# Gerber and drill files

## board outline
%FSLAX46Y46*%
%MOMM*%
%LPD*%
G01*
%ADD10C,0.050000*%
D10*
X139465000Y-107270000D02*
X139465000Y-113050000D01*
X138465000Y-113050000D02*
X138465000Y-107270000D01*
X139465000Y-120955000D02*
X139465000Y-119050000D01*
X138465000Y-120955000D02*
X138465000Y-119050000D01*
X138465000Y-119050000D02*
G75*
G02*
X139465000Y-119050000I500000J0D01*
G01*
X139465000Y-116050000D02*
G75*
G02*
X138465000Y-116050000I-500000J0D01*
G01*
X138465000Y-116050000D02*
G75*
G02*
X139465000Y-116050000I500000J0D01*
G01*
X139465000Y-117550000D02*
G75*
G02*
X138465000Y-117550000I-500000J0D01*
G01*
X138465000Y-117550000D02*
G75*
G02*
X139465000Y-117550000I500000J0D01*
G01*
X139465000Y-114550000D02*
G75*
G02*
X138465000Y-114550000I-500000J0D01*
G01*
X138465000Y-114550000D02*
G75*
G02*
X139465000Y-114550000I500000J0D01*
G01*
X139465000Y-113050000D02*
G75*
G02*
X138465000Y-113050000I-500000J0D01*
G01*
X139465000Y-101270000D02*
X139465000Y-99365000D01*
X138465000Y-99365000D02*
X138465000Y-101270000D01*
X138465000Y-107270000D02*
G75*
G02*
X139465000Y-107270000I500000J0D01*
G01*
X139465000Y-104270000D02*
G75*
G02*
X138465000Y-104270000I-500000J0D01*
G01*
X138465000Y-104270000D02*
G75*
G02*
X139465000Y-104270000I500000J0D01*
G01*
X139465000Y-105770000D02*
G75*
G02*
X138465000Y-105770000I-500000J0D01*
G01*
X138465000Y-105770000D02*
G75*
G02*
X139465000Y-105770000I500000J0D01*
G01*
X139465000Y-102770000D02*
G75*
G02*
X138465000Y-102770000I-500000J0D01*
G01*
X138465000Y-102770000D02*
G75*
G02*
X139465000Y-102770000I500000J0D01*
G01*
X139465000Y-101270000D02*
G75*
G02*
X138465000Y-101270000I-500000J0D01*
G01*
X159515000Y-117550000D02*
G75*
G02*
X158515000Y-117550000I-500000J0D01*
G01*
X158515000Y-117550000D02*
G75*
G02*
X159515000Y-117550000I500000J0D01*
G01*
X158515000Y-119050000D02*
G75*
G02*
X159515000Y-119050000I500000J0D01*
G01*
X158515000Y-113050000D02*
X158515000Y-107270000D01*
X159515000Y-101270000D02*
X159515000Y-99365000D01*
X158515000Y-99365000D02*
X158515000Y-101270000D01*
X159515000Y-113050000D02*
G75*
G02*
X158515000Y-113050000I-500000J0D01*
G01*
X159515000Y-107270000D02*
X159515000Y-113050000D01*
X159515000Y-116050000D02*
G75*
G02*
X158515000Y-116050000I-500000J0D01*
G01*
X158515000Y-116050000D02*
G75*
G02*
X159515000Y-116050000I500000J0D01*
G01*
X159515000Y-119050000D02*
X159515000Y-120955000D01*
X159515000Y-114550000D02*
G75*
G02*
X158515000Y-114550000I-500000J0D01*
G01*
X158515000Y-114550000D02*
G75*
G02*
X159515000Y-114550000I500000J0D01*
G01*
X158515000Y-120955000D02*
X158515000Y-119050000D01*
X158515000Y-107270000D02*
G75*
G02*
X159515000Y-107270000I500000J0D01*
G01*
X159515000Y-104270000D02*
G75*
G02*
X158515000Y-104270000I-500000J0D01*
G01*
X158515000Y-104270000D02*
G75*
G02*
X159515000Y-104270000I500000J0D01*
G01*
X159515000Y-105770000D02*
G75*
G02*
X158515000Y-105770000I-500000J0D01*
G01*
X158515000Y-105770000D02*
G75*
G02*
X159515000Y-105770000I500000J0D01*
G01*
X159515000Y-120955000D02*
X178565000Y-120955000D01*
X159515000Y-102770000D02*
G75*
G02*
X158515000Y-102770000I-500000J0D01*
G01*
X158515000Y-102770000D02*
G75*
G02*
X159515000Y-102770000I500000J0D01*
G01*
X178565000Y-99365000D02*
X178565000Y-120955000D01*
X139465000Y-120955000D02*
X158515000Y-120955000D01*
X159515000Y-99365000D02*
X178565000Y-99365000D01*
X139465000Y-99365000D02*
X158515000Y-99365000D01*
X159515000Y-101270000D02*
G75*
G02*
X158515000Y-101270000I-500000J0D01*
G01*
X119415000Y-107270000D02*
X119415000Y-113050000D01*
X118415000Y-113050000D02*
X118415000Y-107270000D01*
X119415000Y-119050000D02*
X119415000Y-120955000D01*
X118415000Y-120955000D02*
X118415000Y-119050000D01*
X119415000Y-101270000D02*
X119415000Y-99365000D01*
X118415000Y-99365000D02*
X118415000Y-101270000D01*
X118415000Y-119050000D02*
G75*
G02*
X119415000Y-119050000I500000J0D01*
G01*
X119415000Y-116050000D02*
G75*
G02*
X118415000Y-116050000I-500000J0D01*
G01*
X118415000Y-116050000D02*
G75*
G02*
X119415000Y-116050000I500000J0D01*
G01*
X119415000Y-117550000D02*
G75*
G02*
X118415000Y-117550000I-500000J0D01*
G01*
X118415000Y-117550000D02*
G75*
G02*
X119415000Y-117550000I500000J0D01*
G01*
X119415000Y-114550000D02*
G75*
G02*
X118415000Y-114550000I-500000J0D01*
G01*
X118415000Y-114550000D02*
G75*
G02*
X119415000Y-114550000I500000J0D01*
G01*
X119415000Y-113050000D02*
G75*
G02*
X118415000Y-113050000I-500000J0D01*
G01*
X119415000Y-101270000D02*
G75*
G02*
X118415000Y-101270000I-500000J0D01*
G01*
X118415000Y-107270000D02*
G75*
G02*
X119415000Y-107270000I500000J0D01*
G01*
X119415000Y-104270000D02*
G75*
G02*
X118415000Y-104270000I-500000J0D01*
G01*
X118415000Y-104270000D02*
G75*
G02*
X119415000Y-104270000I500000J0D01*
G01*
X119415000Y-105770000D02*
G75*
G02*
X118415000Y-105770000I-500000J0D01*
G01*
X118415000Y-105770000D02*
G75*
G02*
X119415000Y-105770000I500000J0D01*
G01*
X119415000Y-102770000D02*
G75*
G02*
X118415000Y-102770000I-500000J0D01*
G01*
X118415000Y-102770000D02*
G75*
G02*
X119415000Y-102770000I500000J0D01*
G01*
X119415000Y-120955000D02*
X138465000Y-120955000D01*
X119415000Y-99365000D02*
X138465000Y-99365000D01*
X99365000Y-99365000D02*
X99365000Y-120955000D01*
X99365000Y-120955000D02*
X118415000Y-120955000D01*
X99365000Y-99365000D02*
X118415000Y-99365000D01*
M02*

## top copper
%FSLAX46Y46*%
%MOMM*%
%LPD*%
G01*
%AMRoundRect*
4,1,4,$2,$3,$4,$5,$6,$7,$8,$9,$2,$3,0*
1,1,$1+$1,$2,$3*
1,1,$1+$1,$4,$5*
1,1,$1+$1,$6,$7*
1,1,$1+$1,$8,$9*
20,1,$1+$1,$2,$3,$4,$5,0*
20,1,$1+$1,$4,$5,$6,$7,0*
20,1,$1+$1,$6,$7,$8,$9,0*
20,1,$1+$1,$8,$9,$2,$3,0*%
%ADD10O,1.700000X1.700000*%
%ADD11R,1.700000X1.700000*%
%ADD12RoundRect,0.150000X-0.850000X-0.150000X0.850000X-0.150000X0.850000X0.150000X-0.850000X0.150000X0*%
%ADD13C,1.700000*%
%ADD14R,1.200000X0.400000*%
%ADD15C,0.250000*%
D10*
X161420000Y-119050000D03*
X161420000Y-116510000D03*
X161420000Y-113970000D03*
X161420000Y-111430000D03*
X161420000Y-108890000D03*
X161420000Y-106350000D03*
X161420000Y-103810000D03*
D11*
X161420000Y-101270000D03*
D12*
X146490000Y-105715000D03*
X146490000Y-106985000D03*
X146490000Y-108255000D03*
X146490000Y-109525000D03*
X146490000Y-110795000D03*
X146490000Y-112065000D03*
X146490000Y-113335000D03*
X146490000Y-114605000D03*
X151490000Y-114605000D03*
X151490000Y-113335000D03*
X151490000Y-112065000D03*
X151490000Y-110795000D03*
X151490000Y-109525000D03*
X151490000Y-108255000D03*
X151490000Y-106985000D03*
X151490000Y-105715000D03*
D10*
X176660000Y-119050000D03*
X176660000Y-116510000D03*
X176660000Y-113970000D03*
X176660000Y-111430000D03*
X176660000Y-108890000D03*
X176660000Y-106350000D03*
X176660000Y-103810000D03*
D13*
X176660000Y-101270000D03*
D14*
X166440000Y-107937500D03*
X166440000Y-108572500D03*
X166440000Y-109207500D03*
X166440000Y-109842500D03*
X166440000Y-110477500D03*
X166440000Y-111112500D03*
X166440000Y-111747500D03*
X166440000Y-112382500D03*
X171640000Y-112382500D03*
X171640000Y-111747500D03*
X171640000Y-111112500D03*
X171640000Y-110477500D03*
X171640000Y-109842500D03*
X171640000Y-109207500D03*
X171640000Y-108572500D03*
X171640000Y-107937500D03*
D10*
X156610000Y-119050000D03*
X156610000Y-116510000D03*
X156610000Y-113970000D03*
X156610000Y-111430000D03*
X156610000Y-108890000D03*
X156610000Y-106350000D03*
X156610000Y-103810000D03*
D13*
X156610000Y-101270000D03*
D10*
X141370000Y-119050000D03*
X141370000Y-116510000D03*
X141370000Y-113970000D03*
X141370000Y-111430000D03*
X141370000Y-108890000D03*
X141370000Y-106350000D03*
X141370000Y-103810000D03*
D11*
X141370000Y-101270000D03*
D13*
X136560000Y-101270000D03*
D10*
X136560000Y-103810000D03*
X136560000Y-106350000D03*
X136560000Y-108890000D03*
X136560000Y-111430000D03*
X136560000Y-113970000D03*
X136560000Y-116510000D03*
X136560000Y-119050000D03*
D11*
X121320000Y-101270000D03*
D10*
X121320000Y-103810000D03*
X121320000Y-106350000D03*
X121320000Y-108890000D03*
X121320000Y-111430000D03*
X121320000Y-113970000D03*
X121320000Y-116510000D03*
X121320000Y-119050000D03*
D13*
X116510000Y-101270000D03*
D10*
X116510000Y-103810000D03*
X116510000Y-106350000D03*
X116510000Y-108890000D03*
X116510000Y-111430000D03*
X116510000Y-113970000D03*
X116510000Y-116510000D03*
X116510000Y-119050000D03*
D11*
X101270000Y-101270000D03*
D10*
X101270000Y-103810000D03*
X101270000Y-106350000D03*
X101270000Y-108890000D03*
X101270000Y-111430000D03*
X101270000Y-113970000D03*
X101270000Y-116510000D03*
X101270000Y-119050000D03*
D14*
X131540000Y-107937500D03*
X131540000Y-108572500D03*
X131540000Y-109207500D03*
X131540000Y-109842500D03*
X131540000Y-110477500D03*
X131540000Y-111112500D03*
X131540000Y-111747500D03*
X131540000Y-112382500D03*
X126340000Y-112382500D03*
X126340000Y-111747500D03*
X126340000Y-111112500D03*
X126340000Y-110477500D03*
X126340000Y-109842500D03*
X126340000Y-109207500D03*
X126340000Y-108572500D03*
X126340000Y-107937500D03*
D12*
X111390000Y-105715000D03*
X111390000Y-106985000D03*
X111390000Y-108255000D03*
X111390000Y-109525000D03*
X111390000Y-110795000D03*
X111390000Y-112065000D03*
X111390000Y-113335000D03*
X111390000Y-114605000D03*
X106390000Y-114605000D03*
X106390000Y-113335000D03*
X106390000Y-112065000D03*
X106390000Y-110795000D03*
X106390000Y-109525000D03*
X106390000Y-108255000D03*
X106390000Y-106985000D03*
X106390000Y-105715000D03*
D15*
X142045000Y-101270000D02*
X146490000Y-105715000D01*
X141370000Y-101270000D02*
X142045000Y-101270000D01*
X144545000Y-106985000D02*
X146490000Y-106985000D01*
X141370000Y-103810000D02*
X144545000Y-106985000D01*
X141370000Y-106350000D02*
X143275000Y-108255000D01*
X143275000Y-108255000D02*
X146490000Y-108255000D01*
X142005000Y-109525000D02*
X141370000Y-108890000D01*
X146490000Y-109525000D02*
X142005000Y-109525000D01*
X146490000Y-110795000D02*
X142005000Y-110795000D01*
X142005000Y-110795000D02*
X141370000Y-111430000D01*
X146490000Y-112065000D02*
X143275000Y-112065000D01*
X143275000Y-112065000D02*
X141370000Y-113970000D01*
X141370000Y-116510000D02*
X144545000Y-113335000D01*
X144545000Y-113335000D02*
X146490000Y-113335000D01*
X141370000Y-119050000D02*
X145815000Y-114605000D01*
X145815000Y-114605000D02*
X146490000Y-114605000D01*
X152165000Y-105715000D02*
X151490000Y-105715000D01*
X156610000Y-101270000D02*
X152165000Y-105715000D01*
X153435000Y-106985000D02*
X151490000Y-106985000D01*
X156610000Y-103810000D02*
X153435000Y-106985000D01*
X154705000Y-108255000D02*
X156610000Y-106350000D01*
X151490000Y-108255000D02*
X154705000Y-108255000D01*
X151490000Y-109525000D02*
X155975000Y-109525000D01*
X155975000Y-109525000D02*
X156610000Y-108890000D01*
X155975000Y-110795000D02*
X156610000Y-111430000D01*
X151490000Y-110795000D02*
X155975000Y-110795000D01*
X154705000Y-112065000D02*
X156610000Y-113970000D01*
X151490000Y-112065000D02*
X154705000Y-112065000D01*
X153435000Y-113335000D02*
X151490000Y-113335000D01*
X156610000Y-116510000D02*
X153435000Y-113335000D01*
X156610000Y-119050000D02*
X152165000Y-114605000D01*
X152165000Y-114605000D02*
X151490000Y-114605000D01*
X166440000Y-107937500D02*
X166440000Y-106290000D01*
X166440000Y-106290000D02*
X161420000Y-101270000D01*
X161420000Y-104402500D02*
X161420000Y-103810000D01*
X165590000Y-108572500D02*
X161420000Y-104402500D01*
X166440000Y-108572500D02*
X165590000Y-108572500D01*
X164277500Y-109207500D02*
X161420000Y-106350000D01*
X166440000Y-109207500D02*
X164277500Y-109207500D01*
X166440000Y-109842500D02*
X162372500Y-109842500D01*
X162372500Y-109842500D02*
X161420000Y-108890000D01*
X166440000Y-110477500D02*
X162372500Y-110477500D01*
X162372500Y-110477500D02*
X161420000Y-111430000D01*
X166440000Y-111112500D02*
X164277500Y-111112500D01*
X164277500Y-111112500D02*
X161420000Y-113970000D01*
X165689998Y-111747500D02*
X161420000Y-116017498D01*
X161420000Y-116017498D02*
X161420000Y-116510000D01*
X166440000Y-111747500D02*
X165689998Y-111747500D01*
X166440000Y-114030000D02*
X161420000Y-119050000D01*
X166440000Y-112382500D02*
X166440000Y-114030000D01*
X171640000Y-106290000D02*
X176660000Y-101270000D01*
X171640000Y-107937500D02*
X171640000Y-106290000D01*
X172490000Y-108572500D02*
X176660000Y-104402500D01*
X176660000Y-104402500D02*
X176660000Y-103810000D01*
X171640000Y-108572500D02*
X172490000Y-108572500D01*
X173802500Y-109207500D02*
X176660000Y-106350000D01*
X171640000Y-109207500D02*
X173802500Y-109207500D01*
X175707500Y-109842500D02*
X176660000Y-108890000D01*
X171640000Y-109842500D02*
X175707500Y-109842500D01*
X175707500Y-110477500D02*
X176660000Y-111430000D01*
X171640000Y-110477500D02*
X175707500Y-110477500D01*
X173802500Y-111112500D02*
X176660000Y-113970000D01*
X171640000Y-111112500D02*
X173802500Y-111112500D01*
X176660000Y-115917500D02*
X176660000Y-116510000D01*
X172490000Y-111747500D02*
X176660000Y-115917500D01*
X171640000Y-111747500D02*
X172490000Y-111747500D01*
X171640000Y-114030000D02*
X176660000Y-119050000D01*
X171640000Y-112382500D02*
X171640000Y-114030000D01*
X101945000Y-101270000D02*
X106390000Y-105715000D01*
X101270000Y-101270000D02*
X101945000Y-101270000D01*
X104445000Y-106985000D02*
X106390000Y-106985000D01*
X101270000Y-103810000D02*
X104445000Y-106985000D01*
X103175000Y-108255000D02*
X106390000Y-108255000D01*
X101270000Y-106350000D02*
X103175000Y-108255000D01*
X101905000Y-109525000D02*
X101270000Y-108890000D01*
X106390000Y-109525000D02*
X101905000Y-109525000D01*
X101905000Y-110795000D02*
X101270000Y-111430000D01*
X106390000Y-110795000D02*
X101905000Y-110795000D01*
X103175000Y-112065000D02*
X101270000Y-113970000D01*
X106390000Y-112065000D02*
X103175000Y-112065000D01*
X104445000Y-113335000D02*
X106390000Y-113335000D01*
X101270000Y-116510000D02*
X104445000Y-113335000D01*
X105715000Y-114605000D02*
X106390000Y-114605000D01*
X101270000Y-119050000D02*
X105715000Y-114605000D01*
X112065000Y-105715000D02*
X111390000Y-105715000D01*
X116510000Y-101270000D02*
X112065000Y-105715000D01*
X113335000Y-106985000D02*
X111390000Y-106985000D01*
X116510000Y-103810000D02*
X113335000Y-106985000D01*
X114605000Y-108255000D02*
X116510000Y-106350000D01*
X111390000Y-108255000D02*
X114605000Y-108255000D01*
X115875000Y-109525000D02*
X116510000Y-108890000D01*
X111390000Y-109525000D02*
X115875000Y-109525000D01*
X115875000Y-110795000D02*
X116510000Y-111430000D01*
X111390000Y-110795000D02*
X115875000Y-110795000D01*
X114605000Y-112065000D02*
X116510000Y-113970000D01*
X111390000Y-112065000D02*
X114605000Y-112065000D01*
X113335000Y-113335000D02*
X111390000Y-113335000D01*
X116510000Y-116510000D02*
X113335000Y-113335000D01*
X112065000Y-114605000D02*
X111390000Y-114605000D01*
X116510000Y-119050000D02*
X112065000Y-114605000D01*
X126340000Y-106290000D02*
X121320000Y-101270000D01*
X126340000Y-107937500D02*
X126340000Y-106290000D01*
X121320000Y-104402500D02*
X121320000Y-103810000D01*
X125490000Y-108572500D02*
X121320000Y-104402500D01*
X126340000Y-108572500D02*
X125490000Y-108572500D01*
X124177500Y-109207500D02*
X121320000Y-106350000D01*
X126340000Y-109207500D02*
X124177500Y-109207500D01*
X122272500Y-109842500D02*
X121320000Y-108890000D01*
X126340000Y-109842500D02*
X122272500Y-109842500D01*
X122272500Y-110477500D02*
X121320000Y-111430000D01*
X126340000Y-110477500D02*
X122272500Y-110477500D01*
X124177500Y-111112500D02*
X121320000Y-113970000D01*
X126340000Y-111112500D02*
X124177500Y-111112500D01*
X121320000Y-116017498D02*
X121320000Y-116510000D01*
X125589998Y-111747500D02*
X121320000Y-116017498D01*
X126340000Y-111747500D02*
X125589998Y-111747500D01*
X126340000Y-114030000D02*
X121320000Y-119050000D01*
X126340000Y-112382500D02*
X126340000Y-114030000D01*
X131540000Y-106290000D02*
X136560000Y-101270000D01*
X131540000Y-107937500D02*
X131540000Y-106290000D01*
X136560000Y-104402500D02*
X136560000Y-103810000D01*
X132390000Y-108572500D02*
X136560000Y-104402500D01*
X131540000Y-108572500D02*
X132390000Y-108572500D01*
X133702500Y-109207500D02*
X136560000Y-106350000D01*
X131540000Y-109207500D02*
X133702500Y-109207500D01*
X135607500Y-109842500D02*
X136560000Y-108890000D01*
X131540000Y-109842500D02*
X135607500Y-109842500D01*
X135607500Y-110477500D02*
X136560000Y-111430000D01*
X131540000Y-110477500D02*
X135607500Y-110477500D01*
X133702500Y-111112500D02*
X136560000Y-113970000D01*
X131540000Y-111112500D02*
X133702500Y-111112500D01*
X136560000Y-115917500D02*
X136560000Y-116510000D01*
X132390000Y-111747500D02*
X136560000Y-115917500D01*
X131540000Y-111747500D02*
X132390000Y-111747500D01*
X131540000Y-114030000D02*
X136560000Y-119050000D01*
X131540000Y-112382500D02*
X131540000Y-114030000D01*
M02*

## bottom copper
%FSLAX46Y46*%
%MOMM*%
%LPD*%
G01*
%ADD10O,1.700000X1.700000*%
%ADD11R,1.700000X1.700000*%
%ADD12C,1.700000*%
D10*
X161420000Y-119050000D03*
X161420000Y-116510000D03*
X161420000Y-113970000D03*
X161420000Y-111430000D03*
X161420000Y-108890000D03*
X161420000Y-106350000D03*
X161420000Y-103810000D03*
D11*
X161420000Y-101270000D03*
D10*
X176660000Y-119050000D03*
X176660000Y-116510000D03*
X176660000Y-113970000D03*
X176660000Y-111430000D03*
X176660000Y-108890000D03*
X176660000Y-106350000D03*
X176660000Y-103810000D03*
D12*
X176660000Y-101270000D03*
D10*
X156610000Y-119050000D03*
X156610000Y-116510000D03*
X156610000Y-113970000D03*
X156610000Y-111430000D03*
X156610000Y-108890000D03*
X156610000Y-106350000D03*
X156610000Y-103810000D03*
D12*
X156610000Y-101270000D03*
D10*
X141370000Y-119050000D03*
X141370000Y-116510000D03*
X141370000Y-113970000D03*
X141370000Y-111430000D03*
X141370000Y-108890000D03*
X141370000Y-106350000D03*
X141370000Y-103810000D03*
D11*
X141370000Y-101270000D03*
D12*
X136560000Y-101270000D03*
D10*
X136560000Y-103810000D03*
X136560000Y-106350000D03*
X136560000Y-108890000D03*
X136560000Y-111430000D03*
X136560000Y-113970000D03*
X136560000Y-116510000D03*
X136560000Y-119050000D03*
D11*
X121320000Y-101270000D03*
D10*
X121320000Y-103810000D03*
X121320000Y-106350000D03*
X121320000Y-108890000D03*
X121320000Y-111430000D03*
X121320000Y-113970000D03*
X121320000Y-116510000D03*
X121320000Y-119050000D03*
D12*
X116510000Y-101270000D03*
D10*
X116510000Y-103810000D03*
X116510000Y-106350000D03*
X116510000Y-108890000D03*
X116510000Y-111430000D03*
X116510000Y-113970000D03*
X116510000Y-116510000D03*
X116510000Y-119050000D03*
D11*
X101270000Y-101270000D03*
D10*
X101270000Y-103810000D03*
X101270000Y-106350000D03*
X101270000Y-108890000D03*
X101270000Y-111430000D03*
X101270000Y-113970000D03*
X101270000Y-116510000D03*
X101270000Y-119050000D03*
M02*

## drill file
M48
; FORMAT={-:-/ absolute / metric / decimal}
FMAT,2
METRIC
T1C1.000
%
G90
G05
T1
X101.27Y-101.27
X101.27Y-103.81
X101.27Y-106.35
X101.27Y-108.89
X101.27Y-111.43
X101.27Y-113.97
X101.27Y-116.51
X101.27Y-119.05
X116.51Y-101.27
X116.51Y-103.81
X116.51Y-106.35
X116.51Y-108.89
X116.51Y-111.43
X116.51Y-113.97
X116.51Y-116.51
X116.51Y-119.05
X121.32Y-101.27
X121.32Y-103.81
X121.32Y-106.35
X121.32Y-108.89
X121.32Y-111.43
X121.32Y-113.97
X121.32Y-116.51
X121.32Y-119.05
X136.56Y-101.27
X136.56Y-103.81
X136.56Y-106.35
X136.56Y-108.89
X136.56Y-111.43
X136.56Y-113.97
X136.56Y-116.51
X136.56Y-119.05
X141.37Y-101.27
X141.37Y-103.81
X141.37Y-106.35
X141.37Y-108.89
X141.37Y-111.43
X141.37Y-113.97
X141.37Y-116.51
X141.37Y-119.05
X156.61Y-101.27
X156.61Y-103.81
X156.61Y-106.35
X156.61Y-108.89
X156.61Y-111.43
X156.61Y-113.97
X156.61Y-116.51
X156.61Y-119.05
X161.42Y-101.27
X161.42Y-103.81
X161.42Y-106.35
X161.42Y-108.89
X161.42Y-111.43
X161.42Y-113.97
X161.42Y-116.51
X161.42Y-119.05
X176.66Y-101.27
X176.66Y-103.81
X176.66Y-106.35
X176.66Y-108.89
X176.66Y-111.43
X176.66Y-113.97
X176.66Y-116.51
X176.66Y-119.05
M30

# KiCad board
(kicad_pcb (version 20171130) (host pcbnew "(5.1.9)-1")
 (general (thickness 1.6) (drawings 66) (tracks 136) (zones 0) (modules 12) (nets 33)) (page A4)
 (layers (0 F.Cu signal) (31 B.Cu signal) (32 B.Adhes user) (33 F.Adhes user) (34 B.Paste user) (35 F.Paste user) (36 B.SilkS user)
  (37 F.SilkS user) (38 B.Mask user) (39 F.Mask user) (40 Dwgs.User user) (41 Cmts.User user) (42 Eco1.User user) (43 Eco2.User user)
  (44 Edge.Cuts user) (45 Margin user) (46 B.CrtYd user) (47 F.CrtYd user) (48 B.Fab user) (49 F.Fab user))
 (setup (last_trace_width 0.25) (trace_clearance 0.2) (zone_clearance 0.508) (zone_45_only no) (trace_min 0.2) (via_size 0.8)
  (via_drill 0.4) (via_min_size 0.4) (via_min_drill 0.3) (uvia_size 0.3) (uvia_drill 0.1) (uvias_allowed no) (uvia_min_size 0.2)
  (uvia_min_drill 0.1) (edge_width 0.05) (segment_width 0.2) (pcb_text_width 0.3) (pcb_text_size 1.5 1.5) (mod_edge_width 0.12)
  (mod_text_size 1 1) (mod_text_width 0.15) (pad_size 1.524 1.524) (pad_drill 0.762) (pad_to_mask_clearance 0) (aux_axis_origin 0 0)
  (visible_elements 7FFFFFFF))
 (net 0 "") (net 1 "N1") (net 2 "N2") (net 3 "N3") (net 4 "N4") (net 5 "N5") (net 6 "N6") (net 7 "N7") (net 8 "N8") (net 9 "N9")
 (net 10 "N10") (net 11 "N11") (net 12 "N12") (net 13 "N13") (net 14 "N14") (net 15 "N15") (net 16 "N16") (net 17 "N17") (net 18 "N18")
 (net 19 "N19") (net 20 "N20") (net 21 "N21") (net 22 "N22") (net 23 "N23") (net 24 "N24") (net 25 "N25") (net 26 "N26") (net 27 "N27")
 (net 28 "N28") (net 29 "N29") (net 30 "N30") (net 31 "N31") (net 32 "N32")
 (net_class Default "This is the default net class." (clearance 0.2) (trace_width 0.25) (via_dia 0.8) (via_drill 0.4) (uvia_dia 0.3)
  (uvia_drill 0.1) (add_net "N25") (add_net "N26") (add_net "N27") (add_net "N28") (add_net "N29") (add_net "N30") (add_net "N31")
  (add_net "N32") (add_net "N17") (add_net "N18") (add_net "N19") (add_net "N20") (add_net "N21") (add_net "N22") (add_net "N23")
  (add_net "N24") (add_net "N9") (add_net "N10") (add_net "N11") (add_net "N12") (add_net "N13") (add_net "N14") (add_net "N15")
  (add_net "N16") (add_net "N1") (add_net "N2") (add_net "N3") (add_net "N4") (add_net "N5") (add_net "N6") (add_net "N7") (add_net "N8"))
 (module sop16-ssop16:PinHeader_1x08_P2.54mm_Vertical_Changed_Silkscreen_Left (layer B.Cu) (at 161.42 101.27 180)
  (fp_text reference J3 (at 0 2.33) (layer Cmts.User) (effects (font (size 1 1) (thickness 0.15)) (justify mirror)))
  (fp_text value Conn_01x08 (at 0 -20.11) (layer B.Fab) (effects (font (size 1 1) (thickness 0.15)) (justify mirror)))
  (pad 8 thru_hole oval (at 0 -17.78 180) (size 1.7 1.7) (drill 1) (layers *.Cu *.Mask))
  (pad 7 thru_hole oval (at 0 -15.24 180) (size 1.7 1.7) (drill 1) (layers *.Cu *.Mask))
  (pad 6 thru_hole oval (at 0 -12.7 180) (size 1.7 1.7) (drill 1) (layers *.Cu *.Mask))
  (pad 5 thru_hole oval (at 0 -10.16 180) (size 1.7 1.7) (drill 1) (layers *.Cu *.Mask))
  (pad 4 thru_hole oval (at 0 -7.62 180) (size 1.7 1.7) (drill 1) (layers *.Cu *.Mask))
  (pad 3 thru_hole oval (at 0 -5.08 180) (size 1.7 1.7) (drill 1) (layers *.Cu *.Mask))
  (pad 2 thru_hole oval (at 0 -2.54 180) (size 1.7 1.7) (drill 1) (layers *.Cu *.Mask))
  (pad 1 thru_hole rect (at 0 0 180) (size 1.7 1.7) (drill 1) (layers *.Cu *.Mask)))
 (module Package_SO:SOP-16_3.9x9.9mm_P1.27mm (layer F.Cu) (at 148.99 110.16)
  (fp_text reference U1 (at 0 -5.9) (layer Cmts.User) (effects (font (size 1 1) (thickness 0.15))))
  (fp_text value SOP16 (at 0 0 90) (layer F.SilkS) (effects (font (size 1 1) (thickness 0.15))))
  (pad 1 smd roundrect (at -2.5 -4.445) (size 2 0.6) (layers F.Cu F.Paste F.Mask) (roundrect_rratio 0.25))
  (pad 2 smd roundrect (at -2.5 -3.175) (size 2 0.6) (layers F.Cu F.Paste F.Mask) (roundrect_rratio 0.25))
  (pad 3 smd roundrect (at -2.5 -1.905) (size 2 0.6) (layers F.Cu F.Paste F.Mask) (roundrect_rratio 0.25))
  (pad 4 smd roundrect (at -2.5 -0.635) (size 2 0.6) (layers F.Cu F.Paste F.Mask) (roundrect_rratio 0.25))
  (pad 5 smd roundrect (at -2.5 0.635) (size 2 0.6) (layers F.Cu F.Paste F.Mask) (roundrect_rratio 0.25))
  (pad 6 smd roundrect (at -2.5 1.905) (size 2 0.6) (layers F.Cu F.Paste F.Mask) (roundrect_rratio 0.25))
  (pad 7 smd roundrect (at -2.5 3.175) (size 2 0.6) (layers F.Cu F.Paste F.Mask) (roundrect_rratio 0.25))
  (pad 8 smd roundrect (at -2.5 4.445) (size 2 0.6) (layers F.Cu F.Paste F.Mask) (roundrect_rratio 0.25))
  (pad 9 smd roundrect (at 2.5 4.445) (size 2 0.6) (layers F.Cu F.Paste F.Mask) (roundrect_rratio 0.25))
  (pad 10 smd roundrect (at 2.5 3.175) (size 2 0.6) (layers F.Cu F.Paste F.Mask) (roundrect_rratio 0.25))
  (pad 11 smd roundrect (at 2.5 1.905) (size 2 0.6) (layers F.Cu F.Paste F.Mask) (roundrect_rratio 0.25))
  (pad 12 smd roundrect (at 2.5 0.635) (size 2 0.6) (layers F.Cu F.Paste F.Mask) (roundrect_rratio 0.25))
  (pad 13 smd roundrect (at 2.5 -0.635) (size 2 0.6) (layers F.Cu F.Paste F.Mask) (roundrect_rratio 0.25))
  (pad 14 smd roundrect (at 2.5 -1.905) (size 2 0.6) (layers F.Cu F.Paste F.Mask) (roundrect_rratio 0.25))
  (pad 15 smd roundrect (at 2.5 -3.175) (size 2 0.6) (layers F.Cu F.Paste F.Mask) (roundrect_rratio 0.25))
  (pad 16 smd roundrect (at 2.5 -4.445) (size 2 0.6) (layers F.Cu F.Paste F.Mask) (roundrect_rratio 0.25)))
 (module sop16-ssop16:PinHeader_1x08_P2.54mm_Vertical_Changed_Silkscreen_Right (layer B.Cu) (at 176.66 101.27 180)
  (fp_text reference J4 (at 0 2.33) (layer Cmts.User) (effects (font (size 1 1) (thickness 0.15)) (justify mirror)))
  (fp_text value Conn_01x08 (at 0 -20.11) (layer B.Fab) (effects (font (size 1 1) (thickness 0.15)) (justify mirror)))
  (pad 8 thru_hole oval (at 0 -17.78 180) (size 1.7 1.7) (drill 1) (layers *.Cu *.Mask))
  (pad 7 thru_hole oval (at 0 -15.24 180) (size 1.7 1.7) (drill 1) (layers *.Cu *.Mask))
  (pad 6 thru_hole oval (at 0 -12.7 180) (size 1.7 1.7) (drill 1) (layers *.Cu *.Mask))
  (pad 5 thru_hole oval (at 0 -10.16 180) (size 1.7 1.7) (drill 1) (layers *.Cu *.Mask))
  (pad 4 thru_hole oval (at 0 -7.62 180) (size 1.7 1.7) (drill 1) (layers *.Cu *.Mask))
  (pad 3 thru_hole oval (at 0 -5.08 180) (size 1.7 1.7) (drill 1) (layers *.Cu *.Mask))
  (pad 2 thru_hole oval (at 0 -2.54 180) (size 1.7 1.7) (drill 1) (layers *.Cu *.Mask))
  (pad 1 thru_hole circle (at 0 0 180) (size 1.7 1.7) (drill 1) (layers *.Cu *.Mask)))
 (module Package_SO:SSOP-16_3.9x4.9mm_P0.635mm (layer F.Cu) (at 169.04 110.16)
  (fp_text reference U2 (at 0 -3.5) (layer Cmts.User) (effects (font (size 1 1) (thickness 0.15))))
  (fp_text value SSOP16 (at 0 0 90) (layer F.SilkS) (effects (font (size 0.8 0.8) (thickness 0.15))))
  (pad 1 smd rect (at -2.6 -2.2225) (size 1.2 0.4) (layers F.Cu F.Paste F.Mask))
  (pad 2 smd rect (at -2.6 -1.5875) (size 1.2 0.4) (layers F.Cu F.Paste F.Mask))
  (pad 3 smd rect (at -2.6 -0.9525) (size 1.2 0.4) (layers F.Cu F.Paste F.Mask))
  (pad 4 smd rect (at -2.6 -0.3175) (size 1.2 0.4) (layers F.Cu F.Paste F.Mask))
  (pad 5 smd rect (at -2.6 0.3175) (size 1.2 0.4) (layers F.Cu F.Paste F.Mask))
  (pad 6 smd rect (at -2.6 0.9525) (size 1.2 0.4) (layers F.Cu F.Paste F.Mask))
  (pad 7 smd rect (at -2.6 1.5875) (size 1.2 0.4) (layers F.Cu F.Paste F.Mask))
  (pad 8 smd rect (at -2.6 2.2225) (size 1.2 0.4) (layers F.Cu F.Paste F.Mask))
  (pad 9 smd rect (at 2.6 2.2225) (size 1.2 0.4) (layers F.Cu F.Paste F.Mask))
  (pad 10 smd rect (at 2.6 1.5875) (size 1.2 0.4) (layers F.Cu F.Paste F.Mask))
  (pad 11 smd rect (at 2.6 0.9525) (size 1.2 0.4) (layers F.Cu F.Paste F.Mask))
  (pad 12 smd rect (at 2.6 0.3175) (size 1.2 0.4) (layers F.Cu F.Paste F.Mask))
  (pad 13 smd rect (at 2.6 -0.3175) (size 1.2 0.4) (layers F.Cu F.Paste F.Mask))
  (pad 14 smd rect (at 2.6 -0.9525) (size 1.2 0.4) (layers F.Cu F.Paste F.Mask))
  (pad 15 smd rect (at 2.6 -1.5875) (size 1.2 0.4) (layers F.Cu F.Paste F.Mask))
  (pad 16 smd rect (at 2.6 -2.2225) (size 1.2 0.4) (layers F.Cu F.Paste F.Mask)))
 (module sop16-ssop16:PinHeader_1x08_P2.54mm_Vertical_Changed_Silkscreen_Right (layer B.Cu) (at 156.61 101.27 180)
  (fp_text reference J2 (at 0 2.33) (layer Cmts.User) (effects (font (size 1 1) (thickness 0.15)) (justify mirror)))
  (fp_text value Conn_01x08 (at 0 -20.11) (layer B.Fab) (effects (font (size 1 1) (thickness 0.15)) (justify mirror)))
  (pad 8 thru_hole oval (at 0 -17.78 180) (size 1.7 1.7) (drill 1) (layers *.Cu *.Mask))
  (pad 7 thru_hole oval (at 0 -15.24 180) (size 1.7 1.7) (drill 1) (layers *.Cu *.Mask))
  (pad 6 thru_hole oval (at 0 -12.7 180) (size 1.7 1.7) (drill 1) (layers *.Cu *.Mask))
  (pad 5 thru_hole oval (at 0 -10.16 180) (size 1.7 1.7) (drill 1) (layers *.Cu *.Mask))
  (pad 4 thru_hole oval (at 0 -7.62 180) (size 1.7 1.7) (drill 1) (layers *.Cu *.Mask))
  (pad 3 thru_hole oval (at 0 -5.08 180) (size 1.7 1.7) (drill 1) (layers *.Cu *.Mask))
  (pad 2 thru_hole oval (at 0 -2.54 180) (size 1.7 1.7) (drill 1) (layers *.Cu *.Mask))
  (pad 1 thru_hole circle (at 0 0 180) (size 1.7 1.7) (drill 1) (layers *.Cu *.Mask)))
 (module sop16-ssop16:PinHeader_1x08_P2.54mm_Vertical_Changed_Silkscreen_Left (layer B.Cu) (at 141.37 101.27 180)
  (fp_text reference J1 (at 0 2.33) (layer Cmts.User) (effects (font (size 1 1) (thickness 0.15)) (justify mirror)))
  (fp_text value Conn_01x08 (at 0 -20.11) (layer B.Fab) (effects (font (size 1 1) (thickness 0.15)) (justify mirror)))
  (pad 8 thru_hole oval (at 0 -17.78 180) (size 1.7 1.7) (drill 1) (layers *.Cu *.Mask))
  (pad 7 thru_hole oval (at 0 -15.24 180) (size 1.7 1.7) (drill 1) (layers *.Cu *.Mask))
  (pad 6 thru_hole oval (at 0 -12.7 180) (size 1.7 1.7) (drill 1) (layers *.Cu *.Mask))
  (pad 5 thru_hole oval (at 0 -10.16 180) (size 1.7 1.7) (drill 1) (layers *.Cu *.Mask))
  (pad 4 thru_hole oval (at 0 -7.62 180) (size 1.7 1.7) (drill 1) (layers *.Cu *.Mask))
  (pad 3 thru_hole oval (at 0 -5.08 180) (size 1.7 1.7) (drill 1) (layers *.Cu *.Mask))
  (pad 2 thru_hole oval (at 0 -2.54 180) (size 1.7 1.7) (drill 1) (layers *.Cu *.Mask))
  (pad 1 thru_hole rect (at 0 0 180) (size 1.7 1.7) (drill 1) (layers *.Cu *.Mask)))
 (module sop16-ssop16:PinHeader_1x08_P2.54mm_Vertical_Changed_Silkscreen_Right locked (layer B.Cu) (at 136.56 101.27 180)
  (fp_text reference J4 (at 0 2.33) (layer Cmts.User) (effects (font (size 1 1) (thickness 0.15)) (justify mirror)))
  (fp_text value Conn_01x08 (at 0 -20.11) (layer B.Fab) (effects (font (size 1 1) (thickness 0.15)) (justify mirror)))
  (pad 1 thru_hole circle (at 0 0 180) (size 1.7 1.7) (drill 1) (layers *.Cu *.Mask) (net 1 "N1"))
  (pad 2 thru_hole oval (at 0 -2.54 180) (size 1.7 1.7) (drill 1) (layers *.Cu *.Mask) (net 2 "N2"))
  (pad 3 thru_hole oval (at 0 -5.08 180) (size 1.7 1.7) (drill 1) (layers *.Cu *.Mask) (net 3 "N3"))
  (pad 4 thru_hole oval (at 0 -7.62 180) (size 1.7 1.7) (drill 1) (layers *.Cu *.Mask) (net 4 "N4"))
  (pad 5 thru_hole oval (at 0 -10.16 180) (size 1.7 1.7) (drill 1) (layers *.Cu *.Mask) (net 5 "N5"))
  (pad 6 thru_hole oval (at 0 -12.7 180) (size 1.7 1.7) (drill 1) (layers *.Cu *.Mask) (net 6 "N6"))
  (pad 7 thru_hole oval (at 0 -15.24 180) (size 1.7 1.7) (drill 1) (layers *.Cu *.Mask) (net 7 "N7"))
  (pad 8 thru_hole oval (at 0 -17.78 180) (size 1.7 1.7) (drill 1) (layers *.Cu *.Mask) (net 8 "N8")))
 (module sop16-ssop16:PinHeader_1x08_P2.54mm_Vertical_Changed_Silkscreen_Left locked (layer B.Cu) (at 121.32 101.27 180)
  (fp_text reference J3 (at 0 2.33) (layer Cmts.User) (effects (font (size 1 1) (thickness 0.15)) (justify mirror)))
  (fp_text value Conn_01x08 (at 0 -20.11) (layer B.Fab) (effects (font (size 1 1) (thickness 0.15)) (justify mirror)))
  (pad 1 thru_hole rect (at 0 0 180) (size 1.7 1.7) (drill 1) (layers *.Cu *.Mask) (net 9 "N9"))
  (pad 2 thru_hole oval (at 0 -2.54 180) (size 1.7 1.7) (drill 1) (layers *.Cu *.Mask) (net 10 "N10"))
  (pad 3 thru_hole oval (at 0 -5.08 180) (size 1.7 1.7) (drill 1) (layers *.Cu *.Mask) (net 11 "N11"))
  (pad 4 thru_hole oval (at 0 -7.62 180) (size 1.7 1.7) (drill 1) (layers *.Cu *.Mask) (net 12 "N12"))
  (pad 5 thru_hole oval (at 0 -10.16 180) (size 1.7 1.7) (drill 1) (layers *.Cu *.Mask) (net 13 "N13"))
  (pad 6 thru_hole oval (at 0 -12.7 180) (size 1.7 1.7) (drill 1) (layers *.Cu *.Mask) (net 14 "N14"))
  (pad 7 thru_hole oval (at 0 -15.24 180) (size 1.7 1.7) (drill 1) (layers *.Cu *.Mask) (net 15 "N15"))
  (pad 8 thru_hole oval (at 0 -17.78 180) (size 1.7 1.7) (drill 1) (layers *.Cu *.Mask) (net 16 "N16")))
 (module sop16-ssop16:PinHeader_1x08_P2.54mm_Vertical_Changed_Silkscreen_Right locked (layer B.Cu) (at 116.51 101.27 180)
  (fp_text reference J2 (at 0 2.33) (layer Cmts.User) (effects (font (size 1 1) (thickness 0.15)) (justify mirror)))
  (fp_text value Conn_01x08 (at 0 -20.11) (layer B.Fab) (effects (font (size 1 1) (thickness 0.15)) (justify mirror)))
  (pad 1 thru_hole circle (at 0 0 180) (size 1.7 1.7) (drill 1) (layers *.Cu *.Mask) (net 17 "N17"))
  (pad 2 thru_hole oval (at 0 -2.54 180) (size 1.7 1.7) (drill 1) (layers *.Cu *.Mask) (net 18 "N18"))
  (pad 3 thru_hole oval (at 0 -5.08 180) (size 1.7 1.7) (drill 1) (layers *.Cu *.Mask) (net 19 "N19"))
  (pad 4 thru_hole oval (at 0 -7.62 180) (size 1.7 1.7) (drill 1) (layers *.Cu *.Mask) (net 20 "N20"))
  (pad 5 thru_hole oval (at 0 -10.16 180) (size 1.7 1.7) (drill 1) (layers *.Cu *.Mask) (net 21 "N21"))
  (pad 6 thru_hole oval (at 0 -12.7 180) (size 1.7 1.7) (drill 1) (layers *.Cu *.Mask) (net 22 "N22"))
  (pad 7 thru_hole oval (at 0 -15.24 180) (size 1.7 1.7) (drill 1) (layers *.Cu *.Mask) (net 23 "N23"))
  (pad 8 thru_hole oval (at 0 -17.78 180) (size 1.7 1.7) (drill 1) (layers *.Cu *.Mask) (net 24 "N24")))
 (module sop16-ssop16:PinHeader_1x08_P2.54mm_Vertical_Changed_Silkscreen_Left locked (layer B.Cu) (at 101.27 101.27 180)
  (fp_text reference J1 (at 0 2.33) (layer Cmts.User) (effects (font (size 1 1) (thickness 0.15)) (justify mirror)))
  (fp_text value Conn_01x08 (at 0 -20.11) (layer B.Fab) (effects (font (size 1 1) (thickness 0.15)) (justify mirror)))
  (pad 1 thru_hole rect (at 0 0 180) (size 1.7 1.7) (drill 1) (layers *.Cu *.Mask) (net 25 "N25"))
  (pad 2 thru_hole oval (at 0 -2.54 180) (size 1.7 1.7) (drill 1) (layers *.Cu *.Mask) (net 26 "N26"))
  (pad 3 thru_hole oval (at 0 -5.08 180) (size 1.7 1.7) (drill 1) (layers *.Cu *.Mask) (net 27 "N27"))
  (pad 4 thru_hole oval (at 0 -7.62 180) (size 1.7 1.7) (drill 1) (layers *.Cu *.Mask) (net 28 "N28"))
  (pad 5 thru_hole oval (at 0 -10.16 180) (size 1.7 1.7) (drill 1) (layers *.Cu *.Mask) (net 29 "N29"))
  (pad 6 thru_hole oval (at 0 -12.7 180) (size 1.7 1.7) (drill 1) (layers *.Cu *.Mask) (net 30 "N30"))
  (pad 7 thru_hole oval (at 0 -15.24 180) (size 1.7 1.7) (drill 1) (layers *.Cu *.Mask) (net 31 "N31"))
  (pad 8 thru_hole oval (at 0 -17.78 180) (size 1.7 1.7) (drill 1) (layers *.Cu *.Mask) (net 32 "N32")))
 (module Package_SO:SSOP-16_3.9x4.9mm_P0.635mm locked (layer F.Cu) (at 128.94 110.16)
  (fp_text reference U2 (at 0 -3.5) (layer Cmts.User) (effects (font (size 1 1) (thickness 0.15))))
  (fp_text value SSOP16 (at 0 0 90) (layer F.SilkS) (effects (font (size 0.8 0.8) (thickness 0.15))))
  (pad 16 smd rect (at 2.6 -2.2225) (size 1.2 0.4) (layers F.Cu F.Paste F.Mask) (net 1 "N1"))
  (pad 15 smd rect (at 2.6 -1.5875) (size 1.2 0.4) (layers F.Cu F.Paste F.Mask) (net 2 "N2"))
  (pad 14 smd rect (at 2.6 -0.9525) (size 1.2 0.4) (layers F.Cu F.Paste F.Mask) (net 3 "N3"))
  (pad 13 smd rect (at 2.6 -0.3175) (size 1.2 0.4) (layers F.Cu F.Paste F.Mask) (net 4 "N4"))
  (pad 12 smd rect (at 2.6 0.3175) (size 1.2 0.4) (layers F.Cu F.Paste F.Mask) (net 5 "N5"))
  (pad 11 smd rect (at 2.6 0.9525) (size 1.2 0.4) (layers F.Cu F.Paste F.Mask) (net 6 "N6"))
  (pad 10 smd rect (at 2.6 1.5875) (size 1.2 0.4) (layers F.Cu F.Paste F.Mask) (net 7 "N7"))
  (pad 9 smd rect (at 2.6 2.2225) (size 1.2 0.4) (layers F.Cu F.Paste F.Mask) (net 8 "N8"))
  (pad 8 smd rect (at -2.6 2.2225) (size 1.2 0.4) (layers F.Cu F.Paste F.Mask) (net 16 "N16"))
  (pad 7 smd rect (at -2.6 1.5875) (size 1.2 0.4) (layers F.Cu F.Paste F.Mask) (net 15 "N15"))
  (pad 6 smd rect (at -2.6 0.9525) (size 1.2 0.4) (layers F.Cu F.Paste F.Mask) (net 14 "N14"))
  (pad 5 smd rect (at -2.6 0.3175) (size 1.2 0.4) (layers F.Cu F.Paste F.Mask) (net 13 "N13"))
  (pad 4 smd rect (at -2.6 -0.3175) (size 1.2 0.4) (layers F.Cu F.Paste F.Mask) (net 12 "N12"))
  (pad 3 smd rect (at -2.6 -0.9525) (size 1.2 0.4) (layers F.Cu F.Paste F.Mask) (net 11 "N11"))
  (pad 2 smd rect (at -2.6 -1.5875) (size 1.2 0.4) (layers F.Cu F.Paste F.Mask) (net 10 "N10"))
  (pad 1 smd rect (at -2.6 -2.2225) (size 1.2 0.4) (layers F.Cu F.Paste F.Mask) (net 9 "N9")))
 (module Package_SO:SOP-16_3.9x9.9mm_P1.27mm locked (layer F.Cu) (at 108.89 110.16)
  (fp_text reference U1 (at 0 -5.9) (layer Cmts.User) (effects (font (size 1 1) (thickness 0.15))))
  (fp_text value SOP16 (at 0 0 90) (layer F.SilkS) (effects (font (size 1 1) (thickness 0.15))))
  (pad 16 smd roundrect (at 2.5 -4.445) (size 2 0.6) (layers F.Cu F.Paste F.Mask) (roundrect_rratio 0.25) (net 17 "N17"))
  (pad 15 smd roundrect (at 2.5 -3.175) (size 2 0.6) (layers F.Cu F.Paste F.Mask) (roundrect_rratio 0.25) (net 18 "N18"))
  (pad 14 smd roundrect (at 2.5 -1.905) (size 2 0.6) (layers F.Cu F.Paste F.Mask) (roundrect_rratio 0.25) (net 19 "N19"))
  (pad 13 smd roundrect (at 2.5 -0.635) (size 2 0.6) (layers F.Cu F.Paste F.Mask) (roundrect_rratio 0.25) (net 20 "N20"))
  (pad 12 smd roundrect (at 2.5 0.635) (size 2 0.6) (layers F.Cu F.Paste F.Mask) (roundrect_rratio 0.25) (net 21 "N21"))
  (pad 11 smd roundrect (at 2.5 1.905) (size 2 0.6) (layers F.Cu F.Paste F.Mask) (roundrect_rratio 0.25) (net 22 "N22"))
  (pad 10 smd roundrect (at 2.5 3.175) (size 2 0.6) (layers F.Cu F.Paste F.Mask) (roundrect_rratio 0.25) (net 23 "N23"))
  (pad 9 smd roundrect (at 2.5 4.445) (size 2 0.6) (layers F.Cu F.Paste F.Mask) (roundrect_rratio 0.25) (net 24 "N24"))
  (pad 8 smd roundrect (at -2.5 4.445) (size 2 0.6) (layers F.Cu F.Paste F.Mask) (roundrect_rratio 0.25) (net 32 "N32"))
  (pad 7 smd roundrect (at -2.5 3.175) (size 2 0.6) (layers F.Cu F.Paste F.Mask) (roundrect_rratio 0.25) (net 31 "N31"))
  (pad 6 smd roundrect (at -2.5 1.905) (size 2 0.6) (layers F.Cu F.Paste F.Mask) (roundrect_rratio 0.25) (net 30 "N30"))
  (pad 5 smd roundrect (at -2.5 0.635) (size 2 0.6) (layers F.Cu F.Paste F.Mask) (roundrect_rratio 0.25) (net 29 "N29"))
  (pad 4 smd roundrect (at -2.5 -0.635) (size 2 0.6) (layers F.Cu F.Paste F.Mask) (roundrect_rratio 0.25) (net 28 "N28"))
  (pad 3 smd roundrect (at -2.5 -1.905) (size 2 0.6) (layers F.Cu F.Paste F.Mask) (roundrect_rratio 0.25) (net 27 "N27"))
  (pad 2 smd roundrect (at -2.5 -3.175) (size 2 0.6) (layers F.Cu F.Paste F.Mask) (roundrect_rratio 0.25) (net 26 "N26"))
  (pad 1 smd roundrect (at -2.5 -4.445) (size 2 0.6) (layers F.Cu F.Paste F.Mask) (roundrect_rratio 0.25) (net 25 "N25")))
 (gr_line (start 139.465 107.27) (end 139.465 113.05) (layer Edge.Cuts) (width 0.05))
 (gr_line (start 138.465 113.05) (end 138.465 107.27) (layer Edge.Cuts) (width 0.05))
 (gr_line (start 139.465 120.955) (end 139.465 119.05) (layer Edge.Cuts) (width 0.05))
 (gr_line (start 138.465 120.955) (end 138.465 119.05) (layer Edge.Cuts) (width 0.05))
 (gr_arc (start 138.965 119.05) (end 139.465 119.05) (angle -180) (layer Edge.Cuts) (width 0.05))
 (gr_circle (center 138.965 116.05) (end 139.465 116.05) (layer Edge.Cuts) (width 0.05))
 (gr_circle (center 138.965 117.55) (end 139.465 117.55) (layer Edge.Cuts) (width 0.05))
 (gr_circle (center 138.965 114.55) (end 139.465 114.55) (layer Edge.Cuts) (width 0.05))
 (gr_arc (start 138.965 113.05) (end 139.465 113.05) (angle 180) (layer Edge.Cuts) (width 0.05))
 (gr_line (start 139.465 101.27) (end 139.465 99.365) (layer Edge.Cuts) (width 0.05))
 (gr_line (start 138.465 99.365) (end 138.465 101.27) (layer Edge.Cuts) (width 0.05))
 (gr_arc (start 138.965 107.27) (end 139.465 107.27) (angle -180) (layer Edge.Cuts) (width 0.05))
 (gr_circle (center 138.965 104.27) (end 139.465 104.27) (layer Edge.Cuts) (width 0.05))
 (gr_circle (center 138.965 105.77) (end 139.465 105.77) (layer Edge.Cuts) (width 0.05))
 (gr_circle (center 138.965 102.77) (end 139.465 102.77) (layer Edge.Cuts) (width 0.05))
 (gr_arc (start 138.965 101.27) (end 139.465 101.27) (angle 180) (layer Edge.Cuts) (width 0.05))
 (gr_circle (center 159.015 117.55) (end 159.515 117.55) (layer Edge.Cuts) (width 0.05))
 (gr_arc (start 159.015 119.05) (end 159.515 119.05) (angle -180) (layer Edge.Cuts) (width 0.05))
 (gr_line (start 158.515 113.05) (end 158.515 107.27) (layer Edge.Cuts) (width 0.05))
 (gr_line (start 159.515 101.27) (end 159.515 99.365) (layer Edge.Cuts) (width 0.05))
 (gr_line (start 158.515 99.365) (end 158.515 101.27) (layer Edge.Cuts) (width 0.05))
 (gr_arc (start 159.015 113.05) (end 159.515 113.05) (angle 180) (layer Edge.Cuts) (width 0.05))
 (gr_line (start 159.515 107.27) (end 159.515 113.05) (layer Edge.Cuts) (width 0.05))
 (gr_circle (center 159.015 116.05) (end 159.515 116.05) (layer Edge.Cuts) (width 0.05))
 (gr_line (start 159.515 119.05) (end 159.515 120.955) (layer Edge.Cuts) (width 0.05))
 (gr_circle (center 159.015 114.55) (end 159.515 114.55) (layer Edge.Cuts) (width 0.05))
 (gr_line (start 158.515 120.955) (end 158.515 119.05) (layer Edge.Cuts) (width 0.05))
 (gr_arc (start 159.015 107.27) (end 159.515 107.27) (angle -180) (layer Edge.Cuts) (width 0.05))
 (gr_circle (center 159.015 104.27) (end 159.515 104.27) (layer Edge.Cuts) (width 0.05))
 (gr_circle (center 159.015 105.77) (end 159.515 105.77) (layer Edge.Cuts) (width 0.05))
 (gr_line (start 159.515 120.955) (end 178.565 120.955) (layer Edge.Cuts) (width 0.05))
 (gr_circle (center 159.015 102.77) (end 159.515 102.77) (layer Edge.Cuts) (width 0.05))
 (gr_line (start 178.565 99.365) (end 178.565 120.955) (layer Edge.Cuts) (width 0.05))
 (gr_line (start 139.465 120.955) (end 158.515 120.955) (layer Edge.Cuts) (width 0.05))
 (gr_line (start 159.515 99.365) (end 178.565 99.365) (layer Edge.Cuts) (width 0.05))
 (gr_line (start 139.465 99.365) (end 158.515 99.365) (layer Edge.Cuts) (width 0.05))
 (gr_arc (start 159.015 101.27) (end 159.515 101.27) (angle 180) (layer Edge.Cuts) (width 0.05))
 (gr_line (start 119.415 107.27) (end 119.415 113.05) (layer Edge.Cuts) (width 0.05))
 (gr_line (start 118.415 113.05) (end 118.415 107.27) (layer Edge.Cuts) (width 0.05))
 (gr_line (start 119.415 119.05) (end 119.415 120.955) (layer Edge.Cuts) (width 0.05))
 (gr_line (start 118.415 120.955) (end 118.415 119.05) (layer Edge.Cuts) (width 0.05))
 (gr_line (start 119.415 101.27) (end 119.415 99.365) (layer Edge.Cuts) (width 0.05))
 (gr_line (start 118.415 99.365) (end 118.415 101.27) (layer Edge.Cuts) (width 0.05))
 (gr_arc (start 118.915 119.05) (end 119.415 119.05) (angle -180) (layer Edge.Cuts) (width 0.05))
 (gr_circle (center 118.915 116.05) (end 119.415 116.05) (layer Edge.Cuts) (width 0.05))
 (gr_circle (center 118.915 117.55) (end 119.415 117.55) (layer Edge.Cuts) (width 0.05))
 (gr_circle (center 118.915 114.55) (end 119.415 114.55) (layer Edge.Cuts) (width 0.05))
 (gr_arc (start 118.915 113.05) (end 119.415 113.05) (angle 180) (layer Edge.Cuts) (width 0.05))
 (gr_arc (start 118.915 101.27) (end 119.415 101.27) (angle 180) (layer Edge.Cuts) (width 0.05))
 (gr_arc (start 118.915 107.27) (end 119.415 107.27) (angle -180) (layer Edge.Cuts) (width 0.05))
 (gr_circle (center 118.915 104.27) (end 119.415 104.27) (layer Edge.Cuts) (width 0.05))
 (gr_circle (center 118.915 105.77) (end 119.415 105.77) (layer Edge.Cuts) (width 0.05))
 (gr_circle (center 118.915 102.77) (end 119.415 102.77) (layer Edge.Cuts) (width 0.05))
 (gr_line (start 119.415 120.955) (end 138.465 120.955) (layer Edge.Cuts) (width 0.05))
 (gr_line (start 119.415 99.365) (end 138.465 99.365) (layer Edge.Cuts) (width 0.05))
 (gr_line (start 99.365 99.365) (end 99.365 120.955) (layer Edge.Cuts) (width 0.05))
 (gr_line (start 99.365 120.955) (end 118.415 120.955) (layer Edge.Cuts) (width 0.05))
 (gr_line (start 99.365 99.365) (end 118.415 99.365) (layer Edge.Cuts) (width 0.05))
 (segment (start 142.045 101.27) (end 146.49 105.715) (width 0.25) (layer F.Cu) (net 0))
 (segment (start 141.37 101.27) (end 142.045 101.27) (width 0.25) (layer F.Cu) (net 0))
 (segment (start 144.545 106.985) (end 146.49 106.985) (width 0.25) (layer F.Cu) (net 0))
 (segment (start 141.37 103.81) (end 144.545 106.985) (width 0.25) (layer F.Cu) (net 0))
 (segment (start 141.37 106.35) (end 143.275 108.255) (width 0.25) (layer F.Cu) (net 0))
 (segment (start 143.275 108.255) (end 146.49 108.255) (width 0.25) (layer F.Cu) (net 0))
 (segment (start 142.005 109.525) (end 141.37 108.89) (width 0.25) (layer F.Cu) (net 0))
 (segment (start 146.49 109.525) (end 142.005 109.525) (width 0.25) (layer F.Cu) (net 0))
 (segment (start 146.49 110.795) (end 142.005 110.795) (width 0.25) (layer F.Cu) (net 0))
 (segment (start 142.005 110.795) (end 141.37 111.43) (width 0.25) (layer F.Cu) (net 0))
 (segment (start 146.49 112.065) (end 143.275 112.065) (width 0.25) (layer F.Cu) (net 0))
 (segment (start 143.275 112.065) (end 141.37 113.97) (width 0.25) (layer F.Cu) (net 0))
 (segment (start 141.37 116.51) (end 144.545 113.335) (width 0.25) (layer F.Cu) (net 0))
 (segment (start 144.545 113.335) (end 146.49 113.335) (width 0.25) (layer F.Cu) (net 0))
 (segment (start 141.37 119.05) (end 145.815 114.605) (width 0.25) (layer F.Cu) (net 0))
 (segment (start 145.815 114.605) (end 146.49 114.605) (width 0.25) (layer F.Cu) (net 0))
 (segment (start 152.165 105.715) (end 151.49 105.715) (width 0.25) (layer F.Cu) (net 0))
 (segment (start 156.61 101.27) (end 152.165 105.715) (width 0.25) (layer F.Cu) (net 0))
 (segment (start 153.435 106.985) (end 151.49 106.985) (width 0.25) (layer F.Cu) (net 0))
 (segment (start 156.61 103.81) (end 153.435 106.985) (width 0.25) (layer F.Cu) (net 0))
 (segment (start 154.705 108.255) (end 156.61 106.35) (width 0.25) (layer F.Cu) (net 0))
 (segment (start 151.49 108.255) (end 154.705 108.255) (width 0.25) (layer F.Cu) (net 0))
 (segment (start 151.49 109.525) (end 155.975 109.525) (width 0.25) (layer F.Cu) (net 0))
 (segment (start 155.975 109.525) (end 156.61 108.89) (width 0.25) (layer F.Cu) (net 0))
 (segment (start 155.975 110.795) (end 156.61 111.43) (width 0.25) (layer F.Cu) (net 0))
 (segment (start 151.49 110.795) (end 155.975 110.795) (width 0.25) (layer F.Cu) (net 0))
 (segment (start 154.705 112.065) (end 156.61 113.97) (width 0.25) (layer F.Cu) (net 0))
 (segment (start 151.49 112.065) (end 154.705 112.065) (width 0.25) (layer F.Cu) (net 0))
 (segment (start 153.435 113.335) (end 151.49 113.335) (width 0.25) (layer F.Cu) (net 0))
 (segment (start 156.61 116.51) (end 153.435 113.335) (width 0.25) (layer F.Cu) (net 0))
 (segment (start 156.61 119.05) (end 152.165 114.605) (width 0.25) (layer F.Cu) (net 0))
 (segment (start 152.165 114.605) (end 151.49 114.605) (width 0.25) (layer F.Cu) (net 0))
 (segment (start 166.44 107.9375) (end 166.44 106.29) (width 0.25) (layer F.Cu) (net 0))
 (segment (start 166.44 106.29) (end 161.42 101.27) (width 0.25) (layer F.Cu) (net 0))
 (segment (start 161.42 104.4025) (end 161.42 103.81) (width 0.25) (layer F.Cu) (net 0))
 (segment (start 165.59 108.5725) (end 161.42 104.4025) (width 0.25) (layer F.Cu) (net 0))
 (segment (start 166.44 108.5725) (end 165.59 108.5725) (width 0.25) (layer F.Cu) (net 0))
 (segment (start 164.2775 109.2075) (end 161.42 106.35) (width 0.25) (layer F.Cu) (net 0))
 (segment (start 166.44 109.2075) (end 164.2775 109.2075) (width 0.25) (layer F.Cu) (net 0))
 (segment (start 166.44 109.8425) (end 162.3725 109.8425) (width 0.25) (layer F.Cu) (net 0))
 (segment (start 162.3725 109.8425) (end 161.42 108.89) (width 0.25) (layer F.Cu) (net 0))
 (segment (start 166.44 110.4775) (end 162.3725 110.4775) (width 0.25) (layer F.Cu) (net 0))
 (segment (start 162.3725 110.4775) (end 161.42 111.43) (width 0.25) (layer F.Cu) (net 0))
 (segment (start 166.44 111.1125) (end 164.2775 111.1125) (width 0.25) (layer F.Cu) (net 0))
 (segment (start 164.2775 111.1125) (end 161.42 113.97) (width 0.25) (layer F.Cu) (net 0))
 (segment (start 165.689998 111.7475) (end 161.42 116.017498) (width 0.25) (layer F.Cu) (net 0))
 (segment (start 161.42 116.017498) (end 161.42 116.51) (width 0.25) (layer F.Cu) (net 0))
 (segment (start 166.44 111.7475) (end 165.689998 111.7475) (width 0.25) (layer F.Cu) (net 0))
 (segment (start 166.44 114.03) (end 161.42 119.05) (width 0.25) (layer F.Cu) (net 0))
 (segment (start 166.44 112.3825) (end 166.44 114.03) (width 0.25) (layer F.Cu) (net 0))
 (segment (start 171.64 106.29) (end 176.66 101.27) (width 0.25) (layer F.Cu) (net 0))
 (segment (start 171.64 107.9375) (end 171.64 106.29) (width 0.25) (layer F.Cu) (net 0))
 (segment (start 172.49 108.5725) (end 176.66 104.4025) (width 0.25) (layer F.Cu) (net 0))
 (segment (start 176.66 104.4025) (end 176.66 103.81) (width 0.25) (layer F.Cu) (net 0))
 (segment (start 171.64 108.5725) (end 172.49 108.5725) (width 0.25) (layer F.Cu) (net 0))
 (segment (start 173.8025 109.2075) (end 176.66 106.35) (width 0.25) (layer F.Cu) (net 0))
 (segment (start 171.64 109.2075) (end 173.8025 109.2075) (width 0.25) (layer F.Cu) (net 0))
 (segment (start 175.7075 109.8425) (end 176.66 108.89) (width 0.25) (layer F.Cu) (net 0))
 (segment (start 171.64 109.8425) (end 175.7075 109.8425) (width 0.25) (layer F.Cu) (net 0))
 (segment (start 175.7075 110.4775) (end 176.66 111.43) (width 0.25) (layer F.Cu) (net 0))
 (segment (start 171.64 110.4775) (end 175.7075 110.4775) (width 0.25) (layer F.Cu) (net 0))
 (segment (start 173.8025 111.1125) (end 176.66 113.97) (width 0.25) (layer F.Cu) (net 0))
 (segment (start 171.64 111.1125) (end 173.8025 111.1125) (width 0.25) (layer F.Cu) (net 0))
 (segment (start 176.66 115.9175) (end 176.66 116.51) (width 0.25) (layer F.Cu) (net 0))
 (segment (start 172.49 111.7475) (end 176.66 115.9175) (width 0.25) (layer F.Cu) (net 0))
 (segment (start 171.64 111.7475) (end 172.49 111.7475) (width 0.25) (layer F.Cu) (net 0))
 (segment (start 171.64 114.03) (end 176.66 119.05) (width 0.25) (layer F.Cu) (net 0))
 (segment (start 171.64 112.3825) (end 171.64 114.03) (width 0.25) (layer F.Cu) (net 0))
 (segment (start 101.945 101.27) (end 106.39 105.715) (width 0.25) (layer F.Cu) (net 25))
 (segment (start 101.27 101.27) (end 101.945 101.27) (width 0.25) (layer F.Cu) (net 25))
 (segment (start 104.445 106.985) (end 106.39 106.985) (width 0.25) (layer F.Cu) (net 26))
 (segment (start 101.27 103.81) (end 104.445 106.985) (width 0.25) (layer F.Cu) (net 26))
 (segment (start 103.175 108.255) (end 106.39 108.255) (width 0.25) (layer F.Cu) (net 27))
 (segment (start 101.27 106.35) (end 103.175 108.255) (width 0.25) (layer F.Cu) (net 27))
 (segment (start 101.905 109.525) (end 101.27 108.89) (width 0.25) (layer F.Cu) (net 28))
 (segment (start 106.39 109.525) (end 101.905 109.525) (width 0.25) (layer F.Cu) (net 28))
 (segment (start 101.905 110.795) (end 101.27 111.43) (width 0.25) (layer F.Cu) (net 29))
 (segment (start 106.39 110.795) (end 101.905 110.795) (width 0.25) (layer F.Cu) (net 29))
 (segment (start 103.175 112.065) (end 101.27 113.97) (width 0.25) (layer F.Cu) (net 30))
 (segment (start 106.39 112.065) (end 103.175 112.065) (width 0.25) (layer F.Cu) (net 30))
 (segment (start 104.445 113.335) (end 106.39 113.335) (width 0.25) (layer F.Cu) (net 31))
 (segment (start 101.27 116.51) (end 104.445 113.335) (width 0.25) (layer F.Cu) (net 31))
 (segment (start 105.715 114.605) (end 106.39 114.605) (width 0.25) (layer F.Cu) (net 32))
 (segment (start 101.27 119.05) (end 105.715 114.605) (width 0.25) (layer F.Cu) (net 32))
 (segment (start 112.065 105.715) (end 111.39 105.715) (width 0.25) (layer F.Cu) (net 17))
 (segment (start 116.51 101.27) (end 112.065 105.715) (width 0.25) (layer F.Cu) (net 17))
 (segment (start 113.335 106.985) (end 111.39 106.985) (width 0.25) (layer F.Cu) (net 18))
 (segment (start 116.51 103.81) (end 113.335 106.985) (width 0.25) (layer F.Cu) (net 18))
 (segment (start 114.605 108.255) (end 116.51 106.35) (width 0.25) (layer F.Cu) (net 19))
 (segment (start 111.39 108.255) (end 114.605 108.255) (width 0.25) (layer F.Cu) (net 19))
 (segment (start 115.875 109.525) (end 116.51 108.89) (width 0.25) (layer F.Cu) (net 20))
 (segment (start 111.39 109.525) (end 115.875 109.525) (width 0.25) (layer F.Cu) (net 20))
 (segment (start 115.875 110.795) (end 116.51 111.43) (width 0.25) (layer F.Cu) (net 21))
 (segment (start 111.39 110.795) (end 115.875 110.795) (width 0.25) (layer F.Cu) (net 21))
 (segment (start 114.605 112.065) (end 116.51 113.97) (width 0.25) (layer F.Cu) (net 22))
 (segment (start 111.39 112.065) (end 114.605 112.065) (width 0.25) (layer F.Cu) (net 22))
 (segment (start 113.335 113.335) (end 111.39 113.335) (width 0.25) (layer F.Cu) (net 23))
 (segment (start 116.51 116.51) (end 113.335 113.335) (width 0.25) (layer F.Cu) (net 23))
 (segment (start 112.065 114.605) (end 111.39 114.605) (width 0.25) (layer F.Cu) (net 24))
 (segment (start 116.51 119.05) (end 112.065 114.605) (width 0.25) (layer F.Cu) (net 24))
 (segment (start 126.34 106.29) (end 121.32 101.27) (width 0.25) (layer F.Cu) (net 9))
 (segment (start 126.34 107.9375) (end 126.34 106.29) (width 0.25) (layer F.Cu) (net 9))
 (segment (start 121.32 104.4025) (end 121.32 103.81) (width 0.25) (layer F.Cu) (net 10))
 (segment (start 125.49 108.5725) (end 121.32 104.4025) (width 0.25) (layer F.Cu) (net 10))
 (segment (start 126.34 108.5725) (end 125.49 108.5725) (width 0.25) (layer F.Cu) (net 10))
 (segment (start 124.1775 109.2075) (end 121.32 106.35) (width 0.25) (layer F.Cu) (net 11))
 (segment (start 126.34 109.2075) (end 124.1775 109.2075) (width 0.25) (layer F.Cu) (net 11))
 (segment (start 122.2725 109.8425) (end 121.32 108.89) (width 0.25) (layer F.Cu) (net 12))
 (segment (start 126.34 109.8425) (end 122.2725 109.8425) (width 0.25) (layer F.Cu) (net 12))
 (segment (start 122.2725 110.4775) (end 121.32 111.43) (width 0.25) (layer F.Cu) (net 13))
 (segment (start 126.34 110.4775) (end 122.2725 110.4775) (width 0.25) (layer F.Cu) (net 13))
 (segment (start 124.1775 111.1125) (end 121.32 113.97) (width 0.25) (layer F.Cu) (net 14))
 (segment (start 126.34 111.1125) (end 124.1775 111.1125) (width 0.25) (layer F.Cu) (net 14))
 (segment (start 121.32 116.017498) (end 121.32 116.51) (width 0.25) (layer F.Cu) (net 15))
 (segment (start 125.589998 111.7475) (end 121.32 116.017498) (width 0.25) (layer F.Cu) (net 15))
 (segment (start 126.34 111.7475) (end 125.589998 111.7475) (width 0.25) (layer F.Cu) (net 15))
 (segment (start 126.34 114.03) (end 121.32 119.05) (width 0.25) (layer F.Cu) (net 16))
 (segment (start 126.34 112.3825) (end 126.34 114.03) (width 0.25) (layer F.Cu) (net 16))
 (segment (start 131.54 106.29) (end 136.56 101.27) (width 0.25) (layer F.Cu) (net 1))
 (segment (start 131.54 107.9375) (end 131.54 106.29) (width 0.25) (layer F.Cu) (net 1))
 (segment (start 136.56 104.4025) (end 136.56 103.81) (width 0.25) (layer F.Cu) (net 2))
 (segment (start 132.39 108.5725) (end 136.56 104.4025) (width 0.25) (layer F.Cu) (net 2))
 (segment (start 131.54 108.5725) (end 132.39 108.5725) (width 0.25) (layer F.Cu) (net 2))
 (segment (start 133.7025 109.2075) (end 136.56 106.35) (width 0.25) (layer F.Cu) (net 3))
 (segment (start 131.54 109.2075) (end 133.7025 109.2075) (width 0.25) (layer F.Cu) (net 3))
 (segment (start 135.6075 109.8425) (end 136.56 108.89) (width 0.25) (layer F.Cu) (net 4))
 (segment (start 131.54 109.8425) (end 135.6075 109.8425) (width 0.25) (layer F.Cu) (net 4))
 (segment (start 135.6075 110.4775) (end 136.56 111.43) (width 0.25) (layer F.Cu) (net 5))
 (segment (start 131.54 110.4775) (end 135.6075 110.4775) (width 0.25) (layer F.Cu) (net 5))
 (segment (start 133.7025 111.1125) (end 136.56 113.97) (width 0.25) (layer F.Cu) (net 6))
 (segment (start 131.54 111.1125) (end 133.7025 111.1125) (width 0.25) (layer F.Cu) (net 6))
 (segment (start 136.56 115.9175) (end 136.56 116.51) (width 0.25) (layer F.Cu) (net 7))
 (segment (start 132.39 111.7475) (end 136.56 115.9175) (width 0.25) (layer F.Cu) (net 7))
 (segment (start 131.54 111.7475) (end 132.39 111.7475) (width 0.25) (layer F.Cu) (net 7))
 (segment (start 131.54 114.03) (end 136.56 119.05) (width 0.25) (layer F.Cu) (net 8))
 (segment (start 131.54 112.3825) (end 131.54 114.03) (width 0.25) (layer F.Cu) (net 8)))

